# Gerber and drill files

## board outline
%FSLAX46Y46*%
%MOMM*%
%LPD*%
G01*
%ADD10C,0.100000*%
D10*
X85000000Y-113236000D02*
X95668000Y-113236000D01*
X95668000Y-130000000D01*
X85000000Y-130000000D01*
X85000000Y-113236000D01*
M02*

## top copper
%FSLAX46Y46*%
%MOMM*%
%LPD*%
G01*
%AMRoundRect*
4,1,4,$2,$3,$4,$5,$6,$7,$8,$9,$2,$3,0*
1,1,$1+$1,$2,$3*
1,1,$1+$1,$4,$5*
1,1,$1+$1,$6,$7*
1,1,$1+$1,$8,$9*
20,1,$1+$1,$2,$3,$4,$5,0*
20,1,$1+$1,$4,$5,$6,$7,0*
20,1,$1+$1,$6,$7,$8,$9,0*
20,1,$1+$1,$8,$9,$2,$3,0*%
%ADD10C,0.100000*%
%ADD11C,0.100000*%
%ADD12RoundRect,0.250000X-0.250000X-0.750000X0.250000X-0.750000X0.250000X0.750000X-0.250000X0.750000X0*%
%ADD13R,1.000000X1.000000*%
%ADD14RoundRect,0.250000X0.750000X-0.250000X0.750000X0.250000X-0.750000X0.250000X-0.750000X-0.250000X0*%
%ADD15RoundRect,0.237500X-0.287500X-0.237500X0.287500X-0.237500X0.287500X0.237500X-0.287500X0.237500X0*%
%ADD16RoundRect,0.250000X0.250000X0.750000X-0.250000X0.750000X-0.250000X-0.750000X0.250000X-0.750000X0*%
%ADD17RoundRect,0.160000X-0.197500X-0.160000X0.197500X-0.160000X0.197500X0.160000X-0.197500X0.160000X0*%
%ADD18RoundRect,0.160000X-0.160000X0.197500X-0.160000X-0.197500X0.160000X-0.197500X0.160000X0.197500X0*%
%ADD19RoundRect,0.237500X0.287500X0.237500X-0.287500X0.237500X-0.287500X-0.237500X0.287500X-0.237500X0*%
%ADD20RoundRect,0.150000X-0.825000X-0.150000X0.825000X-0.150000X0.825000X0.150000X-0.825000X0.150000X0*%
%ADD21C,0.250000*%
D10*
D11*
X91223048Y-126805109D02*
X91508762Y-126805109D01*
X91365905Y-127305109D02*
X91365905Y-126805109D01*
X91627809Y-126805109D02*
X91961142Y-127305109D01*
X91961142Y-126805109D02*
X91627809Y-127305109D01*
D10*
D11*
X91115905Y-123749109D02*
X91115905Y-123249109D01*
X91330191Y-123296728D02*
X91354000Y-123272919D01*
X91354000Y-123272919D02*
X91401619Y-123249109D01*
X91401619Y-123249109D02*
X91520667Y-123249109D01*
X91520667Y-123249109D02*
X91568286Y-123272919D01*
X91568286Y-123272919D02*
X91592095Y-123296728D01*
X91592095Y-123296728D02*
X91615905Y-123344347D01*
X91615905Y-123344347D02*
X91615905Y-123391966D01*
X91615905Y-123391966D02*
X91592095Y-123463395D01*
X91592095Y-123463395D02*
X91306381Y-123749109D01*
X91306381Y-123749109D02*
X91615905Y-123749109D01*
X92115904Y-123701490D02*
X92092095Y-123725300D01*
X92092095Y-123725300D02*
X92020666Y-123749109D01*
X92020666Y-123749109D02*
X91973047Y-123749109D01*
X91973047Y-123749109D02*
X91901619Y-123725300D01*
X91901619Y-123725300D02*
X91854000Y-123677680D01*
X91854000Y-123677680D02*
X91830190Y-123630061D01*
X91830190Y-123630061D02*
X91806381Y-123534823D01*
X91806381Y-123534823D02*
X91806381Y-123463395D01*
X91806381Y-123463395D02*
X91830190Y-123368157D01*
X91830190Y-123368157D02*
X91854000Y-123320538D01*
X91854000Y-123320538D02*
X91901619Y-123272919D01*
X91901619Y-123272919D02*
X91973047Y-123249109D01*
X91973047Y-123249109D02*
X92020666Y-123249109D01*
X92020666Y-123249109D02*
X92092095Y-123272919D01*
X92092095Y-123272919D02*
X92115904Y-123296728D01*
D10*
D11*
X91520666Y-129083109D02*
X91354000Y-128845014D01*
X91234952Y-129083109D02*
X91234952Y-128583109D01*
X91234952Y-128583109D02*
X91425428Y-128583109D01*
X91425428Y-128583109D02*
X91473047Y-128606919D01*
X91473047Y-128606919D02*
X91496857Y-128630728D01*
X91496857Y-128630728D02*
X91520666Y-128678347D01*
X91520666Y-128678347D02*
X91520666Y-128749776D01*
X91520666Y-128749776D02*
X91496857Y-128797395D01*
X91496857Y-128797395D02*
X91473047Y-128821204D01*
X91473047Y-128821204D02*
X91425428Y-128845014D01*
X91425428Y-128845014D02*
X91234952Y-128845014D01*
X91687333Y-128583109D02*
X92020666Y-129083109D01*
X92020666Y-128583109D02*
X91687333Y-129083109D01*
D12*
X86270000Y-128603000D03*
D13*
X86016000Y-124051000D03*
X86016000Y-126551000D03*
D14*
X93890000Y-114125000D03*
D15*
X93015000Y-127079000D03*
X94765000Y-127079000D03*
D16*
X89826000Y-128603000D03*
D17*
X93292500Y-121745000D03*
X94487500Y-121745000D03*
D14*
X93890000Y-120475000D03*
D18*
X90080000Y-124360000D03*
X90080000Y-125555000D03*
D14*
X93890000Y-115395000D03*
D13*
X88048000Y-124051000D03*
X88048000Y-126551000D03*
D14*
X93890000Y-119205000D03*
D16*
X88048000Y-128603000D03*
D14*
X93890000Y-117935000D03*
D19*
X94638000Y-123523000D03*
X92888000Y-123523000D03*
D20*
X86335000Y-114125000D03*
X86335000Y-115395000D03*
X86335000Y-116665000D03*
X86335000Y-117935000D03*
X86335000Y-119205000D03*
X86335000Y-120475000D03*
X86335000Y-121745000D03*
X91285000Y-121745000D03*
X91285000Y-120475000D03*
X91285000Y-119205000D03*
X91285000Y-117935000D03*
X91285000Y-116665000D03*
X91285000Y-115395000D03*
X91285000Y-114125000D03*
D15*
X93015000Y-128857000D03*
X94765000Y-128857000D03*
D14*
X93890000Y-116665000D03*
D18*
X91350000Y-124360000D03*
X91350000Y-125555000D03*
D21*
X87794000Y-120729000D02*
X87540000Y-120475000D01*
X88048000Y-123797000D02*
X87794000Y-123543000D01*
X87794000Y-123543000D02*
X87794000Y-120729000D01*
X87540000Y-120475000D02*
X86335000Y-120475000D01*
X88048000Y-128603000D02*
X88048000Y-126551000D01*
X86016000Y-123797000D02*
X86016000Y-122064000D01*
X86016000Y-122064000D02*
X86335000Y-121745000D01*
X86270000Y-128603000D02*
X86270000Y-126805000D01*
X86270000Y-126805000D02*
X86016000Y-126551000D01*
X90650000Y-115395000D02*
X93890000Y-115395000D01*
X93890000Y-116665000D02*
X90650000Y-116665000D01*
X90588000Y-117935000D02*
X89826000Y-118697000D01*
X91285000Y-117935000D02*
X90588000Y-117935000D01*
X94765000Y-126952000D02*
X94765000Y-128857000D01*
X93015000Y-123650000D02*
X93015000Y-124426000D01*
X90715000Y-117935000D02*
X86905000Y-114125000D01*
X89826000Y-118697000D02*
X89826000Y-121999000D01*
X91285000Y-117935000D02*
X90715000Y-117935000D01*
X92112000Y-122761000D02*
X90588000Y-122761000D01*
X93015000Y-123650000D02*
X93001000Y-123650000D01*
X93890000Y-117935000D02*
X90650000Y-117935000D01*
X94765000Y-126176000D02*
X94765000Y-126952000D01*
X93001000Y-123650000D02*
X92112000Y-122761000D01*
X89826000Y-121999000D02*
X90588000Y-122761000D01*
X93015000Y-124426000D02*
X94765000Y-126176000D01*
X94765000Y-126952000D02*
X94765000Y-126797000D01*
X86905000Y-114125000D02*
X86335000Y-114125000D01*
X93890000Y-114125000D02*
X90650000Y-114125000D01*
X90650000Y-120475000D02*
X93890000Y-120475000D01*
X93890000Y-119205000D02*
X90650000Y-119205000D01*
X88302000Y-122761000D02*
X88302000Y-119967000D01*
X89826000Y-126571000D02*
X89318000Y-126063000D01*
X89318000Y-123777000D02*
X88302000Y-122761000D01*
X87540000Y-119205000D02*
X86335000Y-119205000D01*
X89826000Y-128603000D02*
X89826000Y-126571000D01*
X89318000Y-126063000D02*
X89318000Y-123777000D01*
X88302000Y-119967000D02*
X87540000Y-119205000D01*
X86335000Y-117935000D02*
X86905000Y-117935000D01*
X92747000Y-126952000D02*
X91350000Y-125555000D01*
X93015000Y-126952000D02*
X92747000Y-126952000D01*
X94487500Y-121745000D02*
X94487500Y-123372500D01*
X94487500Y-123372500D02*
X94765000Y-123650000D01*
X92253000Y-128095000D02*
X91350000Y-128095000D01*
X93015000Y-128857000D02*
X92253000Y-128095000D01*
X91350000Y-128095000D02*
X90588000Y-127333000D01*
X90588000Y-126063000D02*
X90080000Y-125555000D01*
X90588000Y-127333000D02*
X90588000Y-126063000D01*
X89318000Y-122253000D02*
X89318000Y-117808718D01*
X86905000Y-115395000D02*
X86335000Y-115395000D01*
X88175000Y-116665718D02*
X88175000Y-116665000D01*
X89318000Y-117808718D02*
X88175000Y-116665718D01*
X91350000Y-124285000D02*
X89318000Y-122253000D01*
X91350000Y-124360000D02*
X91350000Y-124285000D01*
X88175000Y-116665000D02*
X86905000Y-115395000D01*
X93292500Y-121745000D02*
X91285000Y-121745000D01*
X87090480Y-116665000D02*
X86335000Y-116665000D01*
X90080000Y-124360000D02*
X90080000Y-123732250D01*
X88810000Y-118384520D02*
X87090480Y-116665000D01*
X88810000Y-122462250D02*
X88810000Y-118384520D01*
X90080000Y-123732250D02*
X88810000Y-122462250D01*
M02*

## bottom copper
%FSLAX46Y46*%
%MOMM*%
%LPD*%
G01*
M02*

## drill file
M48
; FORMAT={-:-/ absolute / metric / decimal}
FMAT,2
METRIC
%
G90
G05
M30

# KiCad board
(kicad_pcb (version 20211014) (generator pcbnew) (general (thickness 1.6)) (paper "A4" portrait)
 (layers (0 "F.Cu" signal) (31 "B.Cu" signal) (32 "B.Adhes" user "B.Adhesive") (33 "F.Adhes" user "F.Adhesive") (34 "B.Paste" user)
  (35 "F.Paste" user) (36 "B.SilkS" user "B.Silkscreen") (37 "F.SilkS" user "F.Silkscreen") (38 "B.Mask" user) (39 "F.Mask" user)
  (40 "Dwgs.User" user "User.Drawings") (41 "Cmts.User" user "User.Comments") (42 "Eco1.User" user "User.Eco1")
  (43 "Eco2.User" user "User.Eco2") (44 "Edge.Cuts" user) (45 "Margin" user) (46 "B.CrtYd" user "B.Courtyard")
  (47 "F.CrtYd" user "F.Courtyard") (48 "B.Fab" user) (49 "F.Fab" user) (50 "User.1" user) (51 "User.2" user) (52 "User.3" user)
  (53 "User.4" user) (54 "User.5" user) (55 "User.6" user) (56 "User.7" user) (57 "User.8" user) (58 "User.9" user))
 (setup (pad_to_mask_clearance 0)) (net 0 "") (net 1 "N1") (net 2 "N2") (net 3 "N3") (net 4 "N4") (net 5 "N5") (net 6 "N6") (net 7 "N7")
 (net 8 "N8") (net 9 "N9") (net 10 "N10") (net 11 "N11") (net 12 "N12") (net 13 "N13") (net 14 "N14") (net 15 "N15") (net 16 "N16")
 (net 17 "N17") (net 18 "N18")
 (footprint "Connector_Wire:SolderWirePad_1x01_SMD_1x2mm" (layer "F.Cu") (at 86.27 128.603)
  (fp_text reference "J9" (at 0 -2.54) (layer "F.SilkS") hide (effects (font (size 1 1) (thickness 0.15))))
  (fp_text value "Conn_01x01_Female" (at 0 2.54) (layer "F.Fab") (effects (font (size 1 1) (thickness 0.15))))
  (pad "1" smd roundrect (at 0 0) (size 1 2) (layers "F.Cu" "F.Paste" "F.Mask") (roundrect_rratio 0.25) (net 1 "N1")))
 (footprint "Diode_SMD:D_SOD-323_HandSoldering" (layer "F.Cu") (at 86.016 125.301 -90)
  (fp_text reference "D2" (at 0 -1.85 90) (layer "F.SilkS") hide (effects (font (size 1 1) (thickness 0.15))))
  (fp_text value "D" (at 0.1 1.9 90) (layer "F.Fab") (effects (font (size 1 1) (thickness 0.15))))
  (pad "1" smd rect (at -1.25 0 270) (size 1 1) (layers "F.Cu" "F.Paste" "F.Mask") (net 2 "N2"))
  (pad "2" smd rect (at 1.25 0 270) (size 1 1) (layers "F.Cu" "F.Paste" "F.Mask") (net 1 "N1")))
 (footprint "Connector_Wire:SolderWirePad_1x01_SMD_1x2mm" (layer "F.Cu") (at 93.89 114.125 90)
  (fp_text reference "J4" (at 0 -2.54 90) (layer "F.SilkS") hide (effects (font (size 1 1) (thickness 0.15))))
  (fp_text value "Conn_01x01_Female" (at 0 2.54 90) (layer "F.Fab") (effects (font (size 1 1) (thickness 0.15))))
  (pad "1" smd roundrect (at 0 0 90) (size 1 2) (layers "F.Cu" "F.Paste" "F.Mask") (roundrect_rratio 0.25) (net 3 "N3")))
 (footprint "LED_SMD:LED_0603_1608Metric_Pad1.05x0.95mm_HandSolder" (layer "F.Cu") (at 93.89 127.079)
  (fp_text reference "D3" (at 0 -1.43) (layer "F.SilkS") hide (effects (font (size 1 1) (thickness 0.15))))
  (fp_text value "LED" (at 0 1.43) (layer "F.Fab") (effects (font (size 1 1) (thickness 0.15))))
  (pad "1" smd roundrect (at -0.875 0) (size 1.05 0.95) (layers "F.Cu" "F.Paste" "F.Mask") (roundrect_rratio 0.25) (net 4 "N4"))
  (pad "2" smd roundrect (at 0.875 0) (size 1.05 0.95) (layers "F.Cu" "F.Paste" "F.Mask") (roundrect_rratio 0.25) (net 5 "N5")))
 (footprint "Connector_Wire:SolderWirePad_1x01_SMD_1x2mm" (layer "F.Cu") (at 89.826 128.603 180)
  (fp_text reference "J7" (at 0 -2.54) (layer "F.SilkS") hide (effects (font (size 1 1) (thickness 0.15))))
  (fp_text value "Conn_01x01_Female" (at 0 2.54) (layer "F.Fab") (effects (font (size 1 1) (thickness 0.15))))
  (pad "1" smd roundrect (at 0 0 180) (size 1 2) (layers "F.Cu" "F.Paste" "F.Mask") (roundrect_rratio 0.25) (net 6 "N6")))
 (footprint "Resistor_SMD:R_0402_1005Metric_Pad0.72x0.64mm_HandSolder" (layer "F.Cu") (at 93.89 121.745)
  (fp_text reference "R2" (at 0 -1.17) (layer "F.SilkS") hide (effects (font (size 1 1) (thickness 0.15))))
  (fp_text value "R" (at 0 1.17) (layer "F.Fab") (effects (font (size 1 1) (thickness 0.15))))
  (pad "1" smd roundrect (at -0.5975 0) (size 0.715 0.64) (layers "F.Cu" "F.Paste" "F.Mask") (roundrect_rratio 0.25) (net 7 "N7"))
  (pad "2" smd roundrect (at 0.5975 0) (size 0.715 0.64) (layers "F.Cu" "F.Paste" "F.Mask") (roundrect_rratio 0.25) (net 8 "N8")))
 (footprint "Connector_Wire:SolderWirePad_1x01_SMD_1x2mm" (layer "F.Cu") (at 93.89 120.475 90)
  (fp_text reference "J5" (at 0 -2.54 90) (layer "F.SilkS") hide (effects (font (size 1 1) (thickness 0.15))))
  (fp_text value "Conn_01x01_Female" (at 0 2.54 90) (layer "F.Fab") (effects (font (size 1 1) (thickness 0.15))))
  (pad "1" smd roundrect (at 0 0 90) (size 1 2) (layers "F.Cu" "F.Paste" "F.Mask") (roundrect_rratio 0.25) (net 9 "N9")))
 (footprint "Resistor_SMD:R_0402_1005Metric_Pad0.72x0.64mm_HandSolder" (layer "F.Cu") (at 90.08 124.9575 -90)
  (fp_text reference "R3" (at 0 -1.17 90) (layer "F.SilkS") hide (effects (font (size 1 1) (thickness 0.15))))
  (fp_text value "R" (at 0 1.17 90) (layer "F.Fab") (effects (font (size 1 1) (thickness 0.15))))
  (pad "1" smd roundrect (at -0.5975 0 270) (size 0.715 0.64) (layers "F.Cu" "F.Paste" "F.Mask") (roundrect_rratio 0.25) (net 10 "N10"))
  (pad "2" smd roundrect (at 0.5975 0 270) (size 0.715 0.64) (layers "F.Cu" "F.Paste" "F.Mask") (roundrect_rratio 0.25) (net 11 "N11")))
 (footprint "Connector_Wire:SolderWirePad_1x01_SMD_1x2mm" (layer "F.Cu") (at 93.89 115.395 90)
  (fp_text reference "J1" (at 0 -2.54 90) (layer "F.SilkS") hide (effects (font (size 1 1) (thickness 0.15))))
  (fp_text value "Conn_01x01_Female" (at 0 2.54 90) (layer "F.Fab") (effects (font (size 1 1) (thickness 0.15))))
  (pad "1" smd roundrect (at 0 0 90) (size 1 2) (layers "F.Cu" "F.Paste" "F.Mask") (roundrect_rratio 0.25) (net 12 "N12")))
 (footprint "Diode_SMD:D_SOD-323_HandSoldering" (layer "F.Cu") (at 88.048 125.301 -90)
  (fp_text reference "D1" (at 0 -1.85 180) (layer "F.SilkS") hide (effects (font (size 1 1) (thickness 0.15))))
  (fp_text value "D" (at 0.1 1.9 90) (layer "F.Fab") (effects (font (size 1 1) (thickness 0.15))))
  (pad "1" smd rect (at -1.25 0 270) (size 1 1) (layers "F.Cu" "F.Paste" "F.Mask") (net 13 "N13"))
  (pad "2" smd rect (at 1.25 0 270) (size 1 1) (layers "F.Cu" "F.Paste" "F.Mask") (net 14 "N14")))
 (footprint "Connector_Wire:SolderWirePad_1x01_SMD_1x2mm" (layer "F.Cu") (at 93.89 119.205 90)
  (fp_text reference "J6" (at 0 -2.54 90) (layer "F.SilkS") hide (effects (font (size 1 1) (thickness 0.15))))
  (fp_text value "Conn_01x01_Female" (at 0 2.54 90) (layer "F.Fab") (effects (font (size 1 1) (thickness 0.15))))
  (pad "1" smd roundrect (at 0 0 90) (size 1 2) (layers "F.Cu" "F.Paste" "F.Mask") (roundrect_rratio 0.25) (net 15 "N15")))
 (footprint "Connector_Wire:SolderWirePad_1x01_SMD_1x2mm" (layer "F.Cu") (at 88.048 128.603 180)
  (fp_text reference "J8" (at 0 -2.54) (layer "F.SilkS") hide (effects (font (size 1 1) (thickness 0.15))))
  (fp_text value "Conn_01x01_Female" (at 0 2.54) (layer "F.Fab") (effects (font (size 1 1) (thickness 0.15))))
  (pad "1" smd roundrect (at 0 0 180) (size 1 2) (layers "F.Cu" "F.Paste" "F.Mask") (roundrect_rratio 0.25) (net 14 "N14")))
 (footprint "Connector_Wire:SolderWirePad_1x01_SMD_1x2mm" (layer "F.Cu") (at 93.89 117.935 90)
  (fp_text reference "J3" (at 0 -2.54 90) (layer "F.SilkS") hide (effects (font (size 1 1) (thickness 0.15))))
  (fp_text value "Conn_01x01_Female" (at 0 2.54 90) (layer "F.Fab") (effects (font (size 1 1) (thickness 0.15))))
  (pad "1" smd roundrect (at 0 0 90) (size 1 2) (layers "F.Cu" "F.Paste" "F.Mask") (roundrect_rratio 0.25) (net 5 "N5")))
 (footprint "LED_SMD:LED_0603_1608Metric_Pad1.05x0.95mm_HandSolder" (layer "F.Cu") (at 93.763 123.523 180)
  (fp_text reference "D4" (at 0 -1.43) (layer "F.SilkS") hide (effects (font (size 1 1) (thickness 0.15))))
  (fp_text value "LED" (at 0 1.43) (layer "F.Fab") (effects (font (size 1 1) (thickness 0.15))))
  (pad "1" smd roundrect (at -0.875 0 180) (size 1.05 0.95) (layers "F.Cu" "F.Paste" "F.Mask") (roundrect_rratio 0.25) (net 8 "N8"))
  (pad "2" smd roundrect (at 0.875 0 180) (size 1.05 0.95) (layers "F.Cu" "F.Paste" "F.Mask") (roundrect_rratio 0.25) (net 5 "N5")))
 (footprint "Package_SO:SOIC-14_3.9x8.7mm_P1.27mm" (layer "F.Cu") (at 88.81 117.935)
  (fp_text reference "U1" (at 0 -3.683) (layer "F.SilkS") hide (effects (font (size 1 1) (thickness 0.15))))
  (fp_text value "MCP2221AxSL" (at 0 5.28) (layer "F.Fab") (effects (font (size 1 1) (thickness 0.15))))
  (pad "1" smd roundrect (at -2.475 -3.81) (size 1.95 0.6) (layers "F.Cu" "F.Paste" "F.Mask") (roundrect_rratio 0.25) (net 5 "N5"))
  (pad "2" smd roundrect (at -2.475 -2.54) (size 1.95 0.6) (layers "F.Cu" "F.Paste" "F.Mask") (roundrect_rratio 0.25) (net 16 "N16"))
  (pad "3" smd roundrect (at -2.475 -1.27) (size 1.95 0.6) (layers "F.Cu" "F.Paste" "F.Mask") (roundrect_rratio 0.25) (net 10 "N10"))
  (pad "4" smd roundrect (at -2.475 0) (size 1.95 0.6) (layers "F.Cu" "F.Paste" "F.Mask") (roundrect_rratio 0.25) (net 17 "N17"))
  (pad "5" smd roundrect (at -2.475 1.27) (size 1.95 0.6) (layers "F.Cu" "F.Paste" "F.Mask") (roundrect_rratio 0.25) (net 6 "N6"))
  (pad "6" smd roundrect (at -2.475 2.54) (size 1.95 0.6) (layers "F.Cu" "F.Paste" "F.Mask") (roundrect_rratio 0.25) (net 13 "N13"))
  (pad "7" smd roundrect (at -2.475 3.81) (size 1.95 0.6) (layers "F.Cu" "F.Paste" "F.Mask") (roundrect_rratio 0.25) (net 2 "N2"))
  (pad "8" smd roundrect (at 2.475 3.81) (size 1.95 0.6) (layers "F.Cu" "F.Paste" "F.Mask") (roundrect_rratio 0.25) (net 7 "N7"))
  (pad "9" smd roundrect (at 2.475 2.54) (size 1.95 0.6) (layers "F.Cu" "F.Paste" "F.Mask") (roundrect_rratio 0.25) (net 9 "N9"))
  (pad "10" smd roundrect (at 2.475 1.27) (size 1.95 0.6) (layers "F.Cu" "F.Paste" "F.Mask") (roundrect_rratio 0.25) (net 15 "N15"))
  (pad "11" smd roundrect (at 2.475 0) (size 1.95 0.6) (layers "F.Cu" "F.Paste" "F.Mask") (roundrect_rratio 0.25) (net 5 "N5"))
  (pad "12" smd roundrect (at 2.475 -1.27) (size 1.95 0.6) (layers "F.Cu" "F.Paste" "F.Mask") (roundrect_rratio 0.25) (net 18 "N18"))
  (pad "13" smd roundrect (at 2.475 -2.54) (size 1.95 0.6) (layers "F.Cu" "F.Paste" "F.Mask") (roundrect_rratio 0.25) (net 12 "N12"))
  (pad "14" smd roundrect (at 2.475 -3.81) (size 1.95 0.6) (layers "F.Cu" "F.Paste" "F.Mask") (roundrect_rratio 0.25) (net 3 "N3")))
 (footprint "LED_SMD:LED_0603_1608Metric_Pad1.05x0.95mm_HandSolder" (layer "F.Cu") (at 93.89 128.857)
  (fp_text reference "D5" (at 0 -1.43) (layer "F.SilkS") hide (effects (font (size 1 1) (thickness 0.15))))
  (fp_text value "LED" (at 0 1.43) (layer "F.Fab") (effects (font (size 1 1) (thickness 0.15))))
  (pad "1" smd roundrect (at -0.875 0) (size 1.05 0.95) (layers "F.Cu" "F.Paste" "F.Mask") (roundrect_rratio 0.25) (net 11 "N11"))
  (pad "2" smd roundrect (at 0.875 0) (size 1.05 0.95) (layers "F.Cu" "F.Paste" "F.Mask") (roundrect_rratio 0.25) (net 5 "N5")))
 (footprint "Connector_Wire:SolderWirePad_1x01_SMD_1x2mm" (layer "F.Cu") (at 93.89 116.665 90)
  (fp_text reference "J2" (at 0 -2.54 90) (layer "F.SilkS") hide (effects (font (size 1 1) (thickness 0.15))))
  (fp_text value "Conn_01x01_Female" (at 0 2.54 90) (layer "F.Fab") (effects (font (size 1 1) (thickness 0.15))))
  (pad "1" smd roundrect (at 0 0 90) (size 1 2) (layers "F.Cu" "F.Paste" "F.Mask") (roundrect_rratio 0.25) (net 18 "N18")))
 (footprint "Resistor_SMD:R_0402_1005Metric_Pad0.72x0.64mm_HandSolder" (layer "F.Cu") (at 91.35 124.9575 -90)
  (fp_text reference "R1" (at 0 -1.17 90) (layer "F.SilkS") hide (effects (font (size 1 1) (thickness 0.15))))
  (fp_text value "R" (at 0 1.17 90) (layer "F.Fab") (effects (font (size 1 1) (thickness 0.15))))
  (pad "1" smd roundrect (at -0.5975 0 270) (size 0.715 0.64) (layers "F.Cu" "F.Paste" "F.Mask") (roundrect_rratio 0.25) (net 16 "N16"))
  (pad "2" smd roundrect (at 0.5975 0 270) (size 0.715 0.64) (layers "F.Cu" "F.Paste" "F.Mask") (roundrect_rratio 0.25) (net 4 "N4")))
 (gr_rect (start 95.668 130) (end 85 113.236) (layer "Edge.Cuts") (width 0.1) (fill none))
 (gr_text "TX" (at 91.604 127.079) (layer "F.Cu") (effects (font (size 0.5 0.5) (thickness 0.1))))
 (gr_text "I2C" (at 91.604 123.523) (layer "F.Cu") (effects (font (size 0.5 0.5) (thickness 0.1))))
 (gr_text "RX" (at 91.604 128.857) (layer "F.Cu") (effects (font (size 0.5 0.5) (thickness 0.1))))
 (segment (start 87.794 120.729) (end 87.54 120.475) (width 0.25) (layer "F.Cu") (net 13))
 (segment (start 88.048 123.797) (end 87.794 123.543) (width 0.25) (layer "F.Cu") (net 13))
 (segment (start 87.794 123.543) (end 87.794 120.729) (width 0.25) (layer "F.Cu") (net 13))
 (segment (start 87.54 120.475) (end 86.335 120.475) (width 0.25) (layer "F.Cu") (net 13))
 (segment (start 88.048 128.603) (end 88.048 126.551) (width 0.25) (layer "F.Cu") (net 14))
 (segment (start 86.016 123.797) (end 86.016 122.064) (width 0.25) (layer "F.Cu") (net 2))
 (segment (start 86.016 122.064) (end 86.335 121.745) (width 0.25) (layer "F.Cu") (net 2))
 (segment (start 86.27 128.603) (end 86.27 126.805) (width 0.25) (layer "F.Cu") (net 1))
 (segment (start 86.27 126.805) (end 86.016 126.551) (width 0.25) (layer "F.Cu") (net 1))
 (segment (start 90.65 115.395) (end 93.89 115.395) (width 0.25) (layer "F.Cu") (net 12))
 (segment (start 93.89 116.665) (end 90.65 116.665) (width 0.25) (layer "F.Cu") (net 18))
 (segment (start 90.588 117.935) (end 89.826 118.697) (width 0.25) (layer "F.Cu") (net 5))
 (segment (start 91.285 117.935) (end 90.588 117.935) (width 0.25) (layer "F.Cu") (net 5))
 (segment (start 94.765 126.952) (end 94.765 128.857) (width 0.25) (layer "F.Cu") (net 5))
 (segment (start 93.015 123.65) (end 93.015 124.426) (width 0.25) (layer "F.Cu") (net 5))
 (segment (start 90.715 117.935) (end 86.905 114.125) (width 0.25) (layer "F.Cu") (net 5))
 (segment (start 89.826 118.697) (end 89.826 121.999) (width 0.25) (layer "F.Cu") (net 5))
 (segment (start 91.285 117.935) (end 90.715 117.935) (width 0.25) (layer "F.Cu") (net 5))
 (segment (start 92.112 122.761) (end 90.588 122.761) (width 0.25) (layer "F.Cu") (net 5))
 (segment (start 93.015 123.65) (end 93.001 123.65) (width 0.25) (layer "F.Cu") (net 5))
 (segment (start 93.89 117.935) (end 90.65 117.935) (width 0.25) (layer "F.Cu") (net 5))
 (segment (start 94.765 126.176) (end 94.765 126.952) (width 0.25) (layer "F.Cu") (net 5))
 (segment (start 93.001 123.65) (end 92.112 122.761) (width 0.25) (layer "F.Cu") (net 5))
 (segment (start 89.826 121.999) (end 90.588 122.761) (width 0.25) (layer "F.Cu") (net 5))
 (segment (start 93.015 124.426) (end 94.765 126.176) (width 0.25) (layer "F.Cu") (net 5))
 (segment (start 94.765 126.952) (end 94.765 126.797) (width 0.25) (layer "F.Cu") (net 5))
 (segment (start 86.905 114.125) (end 86.335 114.125) (width 0.25) (layer "F.Cu") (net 5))
 (segment (start 93.89 114.125) (end 90.65 114.125) (width 0.25) (layer "F.Cu") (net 3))
 (segment (start 90.65 120.475) (end 93.89 120.475) (width 0.25) (layer "F.Cu") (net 9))
 (segment (start 93.89 119.205) (end 90.65 119.205) (width 0.25) (layer "F.Cu") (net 15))
 (segment (start 88.302 122.761) (end 88.302 119.967) (width 0.25) (layer "F.Cu") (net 6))
 (segment (start 89.826 126.571) (end 89.318 126.063) (width 0.25) (layer "F.Cu") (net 6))
 (segment (start 89.318 123.777) (end 88.302 122.761) (width 0.25) (layer "F.Cu") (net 6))
 (segment (start 87.54 119.205) (end 86.335 119.205) (width 0.25) (layer "F.Cu") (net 6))
 (segment (start 89.826 128.603) (end 89.826 126.571) (width 0.25) (layer "F.Cu") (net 6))
 (segment (start 89.318 126.063) (end 89.318 123.777) (width 0.25) (layer "F.Cu") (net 6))
 (segment (start 88.302 119.967) (end 87.54 119.205) (width 0.25) (layer "F.Cu") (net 6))
 (segment (start 86.335 117.935) (end 86.905 117.935) (width 0.25) (layer "F.Cu") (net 17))
 (segment (start 92.747 126.952) (end 91.35 125.555) (width 0.25) (layer "F.Cu") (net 4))
 (segment (start 93.015 126.952) (end 92.747 126.952) (width 0.25) (layer "F.Cu") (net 4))
 (segment (start 94.4875 121.745) (end 94.4875 123.3725) (width 0.25) (layer "F.Cu") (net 8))
 (segment (start 94.4875 123.3725) (end 94.765 123.65) (width 0.25) (layer "F.Cu") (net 8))
 (segment (start 92.253 128.095) (end 91.35 128.095) (width 0.25) (layer "F.Cu") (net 11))
 (segment (start 93.015 128.857) (end 92.253 128.095) (width 0.25) (layer "F.Cu") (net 11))
 (segment (start 91.35 128.095) (end 90.588 127.333) (width 0.25) (layer "F.Cu") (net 11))
 (segment (start 90.588 126.063) (end 90.08 125.555) (width 0.25) (layer "F.Cu") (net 11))
 (segment (start 90.588 127.333) (end 90.588 126.063) (width 0.25) (layer "F.Cu") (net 11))
 (segment (start 89.318 122.253) (end 89.318 117.808718) (width 0.25) (layer "F.Cu") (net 16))
 (segment (start 86.905 115.395) (end 86.335 115.395) (width 0.25) (layer "F.Cu") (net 16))
 (segment (start 88.175 116.665718) (end 88.175 116.665) (width 0.25) (layer "F.Cu") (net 16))
 (segment (start 89.318 117.808718) (end 88.175 116.665718) (width 0.25) (layer "F.Cu") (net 16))
 (segment (start 91.35 124.285) (end 89.318 122.253) (width 0.25) (layer "F.Cu") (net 16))
 (segment (start 91.35 124.36) (end 91.35 124.285) (width 0.25) (layer "F.Cu") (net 16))
 (segment (start 88.175 116.665) (end 86.905 115.395) (width 0.25) (layer "F.Cu") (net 16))
 (segment (start 93.2925 121.745) (end 91.285 121.745) (width 0.25) (layer "F.Cu") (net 7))
 (segment (start 87.09048 116.665) (end 86.335 116.665) (width 0.25) (layer "F.Cu") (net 10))
 (segment (start 90.08 124.36) (end 90.08 123.73225) (width 0.25) (layer "F.Cu") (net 10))
 (segment (start 88.81 118.38452) (end 87.09048 116.665) (width 0.25) (layer "F.Cu") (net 10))
 (segment (start 88.81 122.46225) (end 88.81 118.38452) (width 0.25) (layer "F.Cu") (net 10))
 (segment (start 90.08 123.73225) (end 88.81 122.46225) (width 0.25) (layer "F.Cu") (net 10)))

